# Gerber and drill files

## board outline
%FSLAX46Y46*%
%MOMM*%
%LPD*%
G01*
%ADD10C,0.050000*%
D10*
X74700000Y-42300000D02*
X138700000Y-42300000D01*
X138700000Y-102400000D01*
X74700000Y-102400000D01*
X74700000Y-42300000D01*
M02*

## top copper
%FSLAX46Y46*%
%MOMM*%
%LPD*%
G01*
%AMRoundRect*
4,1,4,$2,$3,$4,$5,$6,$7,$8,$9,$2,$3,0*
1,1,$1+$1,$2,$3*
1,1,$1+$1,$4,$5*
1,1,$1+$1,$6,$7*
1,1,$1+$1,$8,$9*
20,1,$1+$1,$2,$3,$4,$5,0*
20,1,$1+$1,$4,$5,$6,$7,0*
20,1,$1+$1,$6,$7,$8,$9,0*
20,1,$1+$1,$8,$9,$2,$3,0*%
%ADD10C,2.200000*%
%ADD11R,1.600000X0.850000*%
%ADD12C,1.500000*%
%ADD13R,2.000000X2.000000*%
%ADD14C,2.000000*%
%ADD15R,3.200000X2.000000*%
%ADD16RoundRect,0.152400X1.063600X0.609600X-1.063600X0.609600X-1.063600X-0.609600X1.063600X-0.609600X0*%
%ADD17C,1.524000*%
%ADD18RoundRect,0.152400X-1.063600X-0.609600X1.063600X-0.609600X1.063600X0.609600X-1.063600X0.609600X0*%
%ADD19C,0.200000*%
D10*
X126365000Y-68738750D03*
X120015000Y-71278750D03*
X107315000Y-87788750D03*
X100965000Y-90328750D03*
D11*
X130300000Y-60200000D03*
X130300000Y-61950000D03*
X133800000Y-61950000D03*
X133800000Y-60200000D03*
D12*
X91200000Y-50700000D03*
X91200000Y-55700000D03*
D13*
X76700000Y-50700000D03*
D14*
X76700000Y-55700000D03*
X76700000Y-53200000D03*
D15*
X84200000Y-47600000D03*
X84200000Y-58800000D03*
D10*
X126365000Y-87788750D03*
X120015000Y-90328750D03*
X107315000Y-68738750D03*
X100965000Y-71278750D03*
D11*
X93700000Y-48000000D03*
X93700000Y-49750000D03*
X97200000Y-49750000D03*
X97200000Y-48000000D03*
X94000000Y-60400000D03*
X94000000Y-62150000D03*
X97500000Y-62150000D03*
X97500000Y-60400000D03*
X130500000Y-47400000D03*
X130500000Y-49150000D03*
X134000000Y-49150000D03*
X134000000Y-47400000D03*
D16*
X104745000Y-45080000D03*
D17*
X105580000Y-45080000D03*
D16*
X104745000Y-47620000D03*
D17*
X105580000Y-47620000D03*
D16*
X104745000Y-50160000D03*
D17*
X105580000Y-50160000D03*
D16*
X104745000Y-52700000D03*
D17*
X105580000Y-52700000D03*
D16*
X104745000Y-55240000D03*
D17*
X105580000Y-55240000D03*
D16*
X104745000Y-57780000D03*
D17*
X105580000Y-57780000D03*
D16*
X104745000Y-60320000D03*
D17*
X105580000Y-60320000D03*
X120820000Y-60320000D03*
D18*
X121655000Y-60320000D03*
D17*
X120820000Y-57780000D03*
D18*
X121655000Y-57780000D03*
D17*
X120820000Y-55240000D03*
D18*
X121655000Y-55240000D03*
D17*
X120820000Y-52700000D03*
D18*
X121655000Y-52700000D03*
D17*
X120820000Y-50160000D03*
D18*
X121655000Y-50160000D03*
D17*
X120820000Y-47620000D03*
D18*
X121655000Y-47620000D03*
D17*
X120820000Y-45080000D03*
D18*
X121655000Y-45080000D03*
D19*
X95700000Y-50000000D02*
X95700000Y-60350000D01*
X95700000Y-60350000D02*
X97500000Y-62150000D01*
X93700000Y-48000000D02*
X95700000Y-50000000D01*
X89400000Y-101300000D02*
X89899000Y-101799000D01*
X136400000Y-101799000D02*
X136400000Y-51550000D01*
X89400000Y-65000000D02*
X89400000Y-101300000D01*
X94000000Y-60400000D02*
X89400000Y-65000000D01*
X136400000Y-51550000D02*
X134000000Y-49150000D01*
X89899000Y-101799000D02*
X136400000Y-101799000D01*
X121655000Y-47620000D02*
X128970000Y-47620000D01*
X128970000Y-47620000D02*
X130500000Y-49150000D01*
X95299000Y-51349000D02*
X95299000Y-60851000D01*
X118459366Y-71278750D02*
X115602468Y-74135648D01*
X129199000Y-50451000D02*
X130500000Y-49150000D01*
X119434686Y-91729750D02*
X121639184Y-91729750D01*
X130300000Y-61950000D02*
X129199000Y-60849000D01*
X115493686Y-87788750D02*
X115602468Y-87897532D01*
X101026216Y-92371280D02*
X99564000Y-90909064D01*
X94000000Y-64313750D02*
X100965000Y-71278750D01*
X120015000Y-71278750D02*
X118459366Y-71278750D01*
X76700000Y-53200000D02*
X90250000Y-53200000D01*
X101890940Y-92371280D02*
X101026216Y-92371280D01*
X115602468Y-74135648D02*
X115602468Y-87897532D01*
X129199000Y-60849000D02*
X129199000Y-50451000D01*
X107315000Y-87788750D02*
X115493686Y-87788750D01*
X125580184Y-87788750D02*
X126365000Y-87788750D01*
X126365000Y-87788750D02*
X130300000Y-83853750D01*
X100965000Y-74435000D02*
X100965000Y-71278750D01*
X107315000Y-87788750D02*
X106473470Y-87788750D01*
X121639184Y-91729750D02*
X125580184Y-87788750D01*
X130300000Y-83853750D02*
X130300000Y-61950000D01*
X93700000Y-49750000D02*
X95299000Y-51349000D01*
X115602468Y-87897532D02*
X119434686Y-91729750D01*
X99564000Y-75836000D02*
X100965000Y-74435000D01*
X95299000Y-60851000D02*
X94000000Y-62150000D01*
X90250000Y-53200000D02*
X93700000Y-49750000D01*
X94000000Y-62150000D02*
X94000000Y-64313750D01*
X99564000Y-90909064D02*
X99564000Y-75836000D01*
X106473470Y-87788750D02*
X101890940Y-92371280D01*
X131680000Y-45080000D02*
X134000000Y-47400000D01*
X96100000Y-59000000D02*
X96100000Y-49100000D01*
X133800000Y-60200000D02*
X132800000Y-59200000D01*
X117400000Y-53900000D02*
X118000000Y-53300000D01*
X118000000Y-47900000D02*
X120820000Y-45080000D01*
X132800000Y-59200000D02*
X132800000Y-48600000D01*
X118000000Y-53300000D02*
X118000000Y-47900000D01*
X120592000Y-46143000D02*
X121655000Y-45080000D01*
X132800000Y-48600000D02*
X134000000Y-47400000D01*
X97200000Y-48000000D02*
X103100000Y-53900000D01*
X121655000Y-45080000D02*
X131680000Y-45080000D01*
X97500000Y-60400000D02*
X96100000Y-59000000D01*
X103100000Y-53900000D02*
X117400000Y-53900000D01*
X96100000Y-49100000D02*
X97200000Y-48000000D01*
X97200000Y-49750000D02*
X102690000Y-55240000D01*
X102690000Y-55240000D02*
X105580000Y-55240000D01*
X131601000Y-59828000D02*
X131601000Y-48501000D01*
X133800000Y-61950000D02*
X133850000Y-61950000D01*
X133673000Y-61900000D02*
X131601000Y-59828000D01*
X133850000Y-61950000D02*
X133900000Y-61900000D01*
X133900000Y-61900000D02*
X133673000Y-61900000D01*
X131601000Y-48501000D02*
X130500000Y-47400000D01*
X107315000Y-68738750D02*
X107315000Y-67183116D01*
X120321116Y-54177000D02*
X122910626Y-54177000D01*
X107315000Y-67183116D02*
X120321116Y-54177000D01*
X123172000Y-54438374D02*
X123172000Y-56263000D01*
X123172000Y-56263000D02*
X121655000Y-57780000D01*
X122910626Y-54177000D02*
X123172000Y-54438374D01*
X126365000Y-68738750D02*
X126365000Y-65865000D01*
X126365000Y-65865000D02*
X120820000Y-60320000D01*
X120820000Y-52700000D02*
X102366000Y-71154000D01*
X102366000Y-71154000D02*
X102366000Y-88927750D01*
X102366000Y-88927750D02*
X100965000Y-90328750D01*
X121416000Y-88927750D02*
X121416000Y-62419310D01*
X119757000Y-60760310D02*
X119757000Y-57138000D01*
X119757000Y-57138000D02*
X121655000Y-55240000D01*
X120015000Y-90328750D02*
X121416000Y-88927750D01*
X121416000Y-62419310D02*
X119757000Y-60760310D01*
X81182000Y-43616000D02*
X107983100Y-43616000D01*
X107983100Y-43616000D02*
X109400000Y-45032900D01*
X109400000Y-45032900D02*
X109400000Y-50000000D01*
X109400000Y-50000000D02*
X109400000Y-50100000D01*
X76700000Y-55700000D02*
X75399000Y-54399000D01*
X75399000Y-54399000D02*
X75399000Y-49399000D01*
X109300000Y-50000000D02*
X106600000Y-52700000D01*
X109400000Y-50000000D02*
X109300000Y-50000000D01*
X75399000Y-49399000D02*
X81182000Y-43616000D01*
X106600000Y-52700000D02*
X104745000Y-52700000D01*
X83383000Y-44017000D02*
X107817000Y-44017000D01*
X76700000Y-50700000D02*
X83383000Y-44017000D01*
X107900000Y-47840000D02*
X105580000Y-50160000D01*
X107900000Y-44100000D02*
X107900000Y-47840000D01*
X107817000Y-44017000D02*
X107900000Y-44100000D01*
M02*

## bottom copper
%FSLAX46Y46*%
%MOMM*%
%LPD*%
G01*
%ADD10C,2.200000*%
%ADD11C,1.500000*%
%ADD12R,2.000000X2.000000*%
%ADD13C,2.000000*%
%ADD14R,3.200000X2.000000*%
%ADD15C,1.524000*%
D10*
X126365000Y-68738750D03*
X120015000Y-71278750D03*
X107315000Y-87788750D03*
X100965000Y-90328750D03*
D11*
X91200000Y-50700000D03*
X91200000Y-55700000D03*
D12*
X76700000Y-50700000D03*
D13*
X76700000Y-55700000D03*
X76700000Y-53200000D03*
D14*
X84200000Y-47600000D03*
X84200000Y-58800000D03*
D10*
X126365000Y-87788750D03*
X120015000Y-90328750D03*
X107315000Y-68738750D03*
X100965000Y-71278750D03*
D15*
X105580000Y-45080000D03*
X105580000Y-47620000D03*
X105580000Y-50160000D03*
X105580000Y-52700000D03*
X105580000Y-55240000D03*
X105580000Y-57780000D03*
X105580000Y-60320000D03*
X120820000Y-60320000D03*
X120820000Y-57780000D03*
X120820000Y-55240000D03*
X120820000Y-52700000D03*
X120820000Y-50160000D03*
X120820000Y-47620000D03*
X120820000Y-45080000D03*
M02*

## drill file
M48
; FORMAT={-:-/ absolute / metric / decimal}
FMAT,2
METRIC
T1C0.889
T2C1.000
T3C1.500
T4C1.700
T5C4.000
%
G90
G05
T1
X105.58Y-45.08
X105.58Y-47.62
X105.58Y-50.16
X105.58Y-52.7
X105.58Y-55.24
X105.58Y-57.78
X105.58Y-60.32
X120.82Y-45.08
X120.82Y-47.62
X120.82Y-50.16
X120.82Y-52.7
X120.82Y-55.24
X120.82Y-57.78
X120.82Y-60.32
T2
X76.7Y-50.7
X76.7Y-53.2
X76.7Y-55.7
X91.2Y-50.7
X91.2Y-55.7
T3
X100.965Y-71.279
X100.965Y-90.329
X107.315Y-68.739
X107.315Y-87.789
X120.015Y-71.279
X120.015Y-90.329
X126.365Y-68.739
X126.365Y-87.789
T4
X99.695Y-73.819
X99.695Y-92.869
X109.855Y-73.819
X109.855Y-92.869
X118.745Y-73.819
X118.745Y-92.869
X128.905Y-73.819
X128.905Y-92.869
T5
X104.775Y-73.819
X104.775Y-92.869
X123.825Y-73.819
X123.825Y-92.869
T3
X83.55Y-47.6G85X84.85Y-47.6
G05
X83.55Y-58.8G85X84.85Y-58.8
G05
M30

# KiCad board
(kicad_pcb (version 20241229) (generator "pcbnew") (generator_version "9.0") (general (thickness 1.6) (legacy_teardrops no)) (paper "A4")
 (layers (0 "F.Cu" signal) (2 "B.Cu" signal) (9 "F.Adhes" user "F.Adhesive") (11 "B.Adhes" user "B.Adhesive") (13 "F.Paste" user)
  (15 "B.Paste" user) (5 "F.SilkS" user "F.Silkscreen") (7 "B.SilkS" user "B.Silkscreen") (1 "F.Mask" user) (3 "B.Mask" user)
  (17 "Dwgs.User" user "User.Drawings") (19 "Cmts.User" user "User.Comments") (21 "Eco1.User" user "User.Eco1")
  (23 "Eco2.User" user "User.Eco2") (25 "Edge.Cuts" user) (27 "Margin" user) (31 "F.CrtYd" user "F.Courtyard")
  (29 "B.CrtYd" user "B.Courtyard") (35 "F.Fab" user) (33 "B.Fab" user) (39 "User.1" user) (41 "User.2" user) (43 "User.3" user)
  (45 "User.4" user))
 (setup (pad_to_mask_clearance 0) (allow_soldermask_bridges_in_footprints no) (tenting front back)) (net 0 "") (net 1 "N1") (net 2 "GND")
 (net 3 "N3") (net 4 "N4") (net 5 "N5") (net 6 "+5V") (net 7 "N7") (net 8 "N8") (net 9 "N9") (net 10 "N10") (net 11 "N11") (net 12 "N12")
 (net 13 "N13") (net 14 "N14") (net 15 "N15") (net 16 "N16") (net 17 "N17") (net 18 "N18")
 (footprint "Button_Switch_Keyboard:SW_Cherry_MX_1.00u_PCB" (layer "F.Cu") (at 126.365 68.73875)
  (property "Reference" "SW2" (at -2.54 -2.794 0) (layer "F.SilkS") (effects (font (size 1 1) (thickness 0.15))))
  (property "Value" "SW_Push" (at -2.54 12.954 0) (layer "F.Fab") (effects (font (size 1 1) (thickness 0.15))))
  (pad "" np_thru_hole circle (at -7.62 5.08) (size 1.7 1.7) (drill 1.7) (layers "*.Cu" "*.Mask"))
  (pad "" np_thru_hole circle (at -2.54 5.08) (size 4 4) (drill 4) (layers "*.Cu" "*.Mask"))
  (pad "" np_thru_hole circle (at 2.54 5.08) (size 1.7 1.7) (drill 1.7) (layers "*.Cu" "*.Mask"))
  (pad "1" thru_hole circle (at 0 0) (size 2.2 2.2) (drill 1.5) (layers "*.Cu" "*.Mask") (remove_unused_layers no) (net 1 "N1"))
  (pad "2" thru_hole circle (at -6.35 2.54) (size 2.2 2.2) (drill 1.5) (layers "*.Cu" "*.Mask") (remove_unused_layers no) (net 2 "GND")))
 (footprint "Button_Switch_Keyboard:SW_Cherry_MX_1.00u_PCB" (layer "F.Cu") (at 107.315 87.78875)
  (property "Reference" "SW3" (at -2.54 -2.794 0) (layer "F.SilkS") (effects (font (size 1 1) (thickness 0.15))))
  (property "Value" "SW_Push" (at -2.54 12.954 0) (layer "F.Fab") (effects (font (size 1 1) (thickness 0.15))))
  (pad "" np_thru_hole circle (at -7.62 5.08) (size 1.7 1.7) (drill 1.7) (layers "*.Cu" "*.Mask"))
  (pad "" np_thru_hole circle (at -2.54 5.08) (size 4 4) (drill 4) (layers "*.Cu" "*.Mask"))
  (pad "" np_thru_hole circle (at 2.54 5.08) (size 1.7 1.7) (drill 1.7) (layers "*.Cu" "*.Mask"))
  (pad "1" thru_hole circle (at 0 0) (size 2.2 2.2) (drill 1.5) (layers "*.Cu" "*.Mask") (remove_unused_layers no) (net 2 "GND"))
  (pad "2" thru_hole circle (at -6.35 2.54) (size 2.2 2.2) (drill 1.5) (layers "*.Cu" "*.Mask") (remove_unused_layers no) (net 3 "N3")))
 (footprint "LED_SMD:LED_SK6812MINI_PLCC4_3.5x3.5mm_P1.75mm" (layer "F.Cu") (at 132.05 61.075)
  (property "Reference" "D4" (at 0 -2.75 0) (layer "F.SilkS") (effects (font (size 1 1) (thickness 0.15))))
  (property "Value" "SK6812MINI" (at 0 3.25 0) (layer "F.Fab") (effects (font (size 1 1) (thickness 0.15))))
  (pad "1" smd rect (at -1.75 -0.875) (size 1.6 0.85) (layers "F.Cu" "F.Mask" "F.Paste") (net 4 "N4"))
  (pad "2" smd rect (at -1.75 0.875) (size 1.6 0.85) (layers "F.Cu" "F.Mask" "F.Paste") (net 2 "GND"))
  (pad "3" smd rect (at 1.75 0.875) (size 1.6 0.85) (layers "F.Cu" "F.Mask" "F.Paste") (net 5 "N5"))
  (pad "4" smd rect (at 1.75 -0.875) (size 1.6 0.85) (layers "F.Cu" "F.Mask" "F.Paste") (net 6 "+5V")))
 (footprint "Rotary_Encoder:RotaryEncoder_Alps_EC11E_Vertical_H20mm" (layer "F.Cu") (at 76.7 50.7)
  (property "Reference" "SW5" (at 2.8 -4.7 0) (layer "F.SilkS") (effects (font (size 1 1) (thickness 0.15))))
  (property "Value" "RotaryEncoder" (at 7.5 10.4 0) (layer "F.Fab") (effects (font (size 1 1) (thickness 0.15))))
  (pad "" thru_hole circle (at 14.5 0) (size 1.5 1.5) (drill 1) (layers "*.Cu" "*.Mask") (remove_unused_layers no))
  (pad "" thru_hole circle (at 14.5 5) (size 1.5 1.5) (drill 1) (layers "*.Cu" "*.Mask") (remove_unused_layers no))
  (pad "A" thru_hole rect (at 0 0) (size 2 2) (drill 1) (layers "*.Cu" "*.Mask") (remove_unused_layers no) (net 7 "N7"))
  (pad "B" thru_hole circle (at 0 5) (size 2 2) (drill 1) (layers "*.Cu" "*.Mask") (remove_unused_layers no) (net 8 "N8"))
  (pad "C" thru_hole circle (at 0 2.5) (size 2 2) (drill 1) (layers "*.Cu" "*.Mask") (remove_unused_layers no) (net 2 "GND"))
  (pad "MP" thru_hole rect (at 7.5 -3.1) (size 3.2 2) (drill oval 2.8 1.5) (layers "*.Cu" "*.Mask") (remove_unused_layers no))
  (pad "MP" thru_hole rect (at 7.5 8.1) (size 3.2 2) (drill oval 2.8 1.5) (layers "*.Cu" "*.Mask") (remove_unused_layers no)))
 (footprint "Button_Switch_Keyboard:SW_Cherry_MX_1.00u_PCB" (layer "F.Cu") (at 126.365 87.78875)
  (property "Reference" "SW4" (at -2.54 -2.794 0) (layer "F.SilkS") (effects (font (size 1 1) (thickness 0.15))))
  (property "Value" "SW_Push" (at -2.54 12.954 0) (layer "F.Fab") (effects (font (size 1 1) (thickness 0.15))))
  (pad "" np_thru_hole circle (at -7.62 5.08) (size 1.7 1.7) (drill 1.7) (layers "*.Cu" "*.Mask"))
  (pad "" np_thru_hole circle (at -2.54 5.08) (size 4 4) (drill 4) (layers "*.Cu" "*.Mask"))
  (pad "" np_thru_hole circle (at 2.54 5.08) (size 1.7 1.7) (drill 1.7) (layers "*.Cu" "*.Mask"))
  (pad "1" thru_hole circle (at 0 0) (size 2.2 2.2) (drill 1.5) (layers "*.Cu" "*.Mask") (remove_unused_layers no) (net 2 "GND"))
  (pad "2" thru_hole circle (at -6.35 2.54) (size 2.2 2.2) (drill 1.5) (layers "*.Cu" "*.Mask") (remove_unused_layers no) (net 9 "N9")))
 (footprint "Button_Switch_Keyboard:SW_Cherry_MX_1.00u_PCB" (layer "F.Cu") (at 107.315 68.73875)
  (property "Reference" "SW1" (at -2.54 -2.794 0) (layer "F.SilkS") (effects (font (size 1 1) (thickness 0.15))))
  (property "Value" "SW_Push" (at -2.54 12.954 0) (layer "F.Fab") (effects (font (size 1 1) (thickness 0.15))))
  (pad "" np_thru_hole circle (at -7.62 5.08) (size 1.7 1.7) (drill 1.7) (layers "*.Cu" "*.Mask"))
  (pad "" np_thru_hole circle (at -2.54 5.08) (size 4 4) (drill 4) (layers "*.Cu" "*.Mask"))
  (pad "" np_thru_hole circle (at 2.54 5.08) (size 1.7 1.7) (drill 1.7) (layers "*.Cu" "*.Mask"))
  (pad "1" thru_hole circle (at 0 0) (size 2.2 2.2) (drill 1.5) (layers "*.Cu" "*.Mask") (remove_unused_layers no) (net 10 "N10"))
  (pad "2" thru_hole circle (at -6.35 2.54) (size 2.2 2.2) (drill 1.5) (layers "*.Cu" "*.Mask") (remove_unused_layers no) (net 2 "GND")))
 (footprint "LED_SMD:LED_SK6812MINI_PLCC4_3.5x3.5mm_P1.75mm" (layer "F.Cu") (at 95.45 48.875)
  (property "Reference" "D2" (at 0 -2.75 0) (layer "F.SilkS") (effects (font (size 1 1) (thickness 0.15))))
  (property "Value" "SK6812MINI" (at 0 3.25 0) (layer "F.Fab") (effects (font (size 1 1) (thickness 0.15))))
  (pad "1" smd rect (at -1.75 -0.875) (size 1.6 0.85) (layers "F.Cu" "F.Mask" "F.Paste") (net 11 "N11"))
  (pad "2" smd rect (at -1.75 0.875) (size 1.6 0.85) (layers "F.Cu" "F.Mask" "F.Paste") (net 2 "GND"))
  (pad "3" smd rect (at 1.75 0.875) (size 1.6 0.85) (layers "F.Cu" "F.Mask" "F.Paste") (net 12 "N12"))
  (pad "4" smd rect (at 1.75 -0.875) (size 1.6 0.85) (layers "F.Cu" "F.Mask" "F.Paste") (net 6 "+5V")))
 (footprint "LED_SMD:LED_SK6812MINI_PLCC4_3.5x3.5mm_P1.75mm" (layer "F.Cu") (at 95.75 61.275)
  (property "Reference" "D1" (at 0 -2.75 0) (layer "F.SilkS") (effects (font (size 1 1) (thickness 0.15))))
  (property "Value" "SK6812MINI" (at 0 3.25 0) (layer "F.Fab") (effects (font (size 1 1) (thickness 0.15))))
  (pad "1" smd rect (at -1.75 -0.875) (size 1.6 0.85) (layers "F.Cu" "F.Mask" "F.Paste") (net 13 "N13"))
  (pad "2" smd rect (at -1.75 0.875) (size 1.6 0.85) (layers "F.Cu" "F.Mask" "F.Paste") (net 2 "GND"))
  (pad "3" smd rect (at 1.75 0.875) (size 1.6 0.85) (layers "F.Cu" "F.Mask" "F.Paste") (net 11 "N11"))
  (pad "4" smd rect (at 1.75 -0.875) (size 1.6 0.85) (layers "F.Cu" "F.Mask" "F.Paste") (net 6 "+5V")))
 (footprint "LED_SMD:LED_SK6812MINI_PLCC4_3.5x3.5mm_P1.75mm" (layer "F.Cu") (at 132.25 48.275)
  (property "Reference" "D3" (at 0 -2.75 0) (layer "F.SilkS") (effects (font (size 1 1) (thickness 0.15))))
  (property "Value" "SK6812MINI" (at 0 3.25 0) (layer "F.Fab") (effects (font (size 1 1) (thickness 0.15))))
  (pad "1" smd rect (at -1.75 -0.875) (size 1.6 0.85) (layers "F.Cu" "F.Mask" "F.Paste") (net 5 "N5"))
  (pad "2" smd rect (at -1.75 0.875) (size 1.6 0.85) (layers "F.Cu" "F.Mask" "F.Paste") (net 2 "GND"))
  (pad "3" smd rect (at 1.75 0.875) (size 1.6 0.85) (layers "F.Cu" "F.Mask" "F.Paste") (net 13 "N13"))
  (pad "4" smd rect (at 1.75 -0.875) (size 1.6 0.85) (layers "F.Cu" "F.Mask" "F.Paste") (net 6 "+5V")))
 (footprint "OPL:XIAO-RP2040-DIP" (layer "F.Cu") (at 113.2 52.7)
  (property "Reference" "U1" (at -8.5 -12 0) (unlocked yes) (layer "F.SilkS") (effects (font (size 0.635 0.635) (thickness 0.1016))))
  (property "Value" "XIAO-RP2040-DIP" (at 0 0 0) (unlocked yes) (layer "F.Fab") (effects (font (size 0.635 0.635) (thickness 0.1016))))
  (pad "1" smd roundrect (at -8.455 -7.62 180) (size 2.432 1.524) (layers "F.Cu" "F.Mask") (roundrect_rratio 0.1) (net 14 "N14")
   (thermal_bridge_angle 45))
  (pad "1" thru_hole circle (at -7.62 -7.62 180) (size 1.524 1.524) (drill 0.889) (layers "*.Cu" "*.Mask") (remove_unused_layers no)
   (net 14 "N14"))
  (pad "2" smd roundrect (at -8.455 -5.08 180) (size 2.432 1.524) (layers "F.Cu" "F.Mask") (roundrect_rratio 0.1) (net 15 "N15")
   (thermal_bridge_angle 45))
  (pad "2" thru_hole circle (at -7.62 -5.08 180) (size 1.524 1.524) (drill 0.889) (layers "*.Cu" "*.Mask") (remove_unused_layers no)
   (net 15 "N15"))
  (pad "3" smd roundrect (at -8.455 -2.54 180) (size 2.432 1.524) (layers "F.Cu" "F.Mask") (roundrect_rratio 0.1) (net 7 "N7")
   (thermal_bridge_angle 45))
  (pad "3" thru_hole circle (at -7.62 -2.54 180) (size 1.524 1.524) (drill 0.889) (layers "*.Cu" "*.Mask") (remove_unused_layers no)
   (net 7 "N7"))
  (pad "4" smd roundrect (at -8.455 0 180) (size 2.432 1.524) (layers "F.Cu" "F.Mask") (roundrect_rratio 0.1) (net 8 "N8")
   (thermal_bridge_angle 45))
  (pad "4" thru_hole circle (at -7.62 0 180) (size 1.524 1.524) (drill 0.889) (layers "*.Cu" "*.Mask") (remove_unused_layers no)
   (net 8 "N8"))
  (pad "5" smd roundrect (at -8.455 2.54 180) (size 2.432 1.524) (layers "F.Cu" "F.Mask") (roundrect_rratio 0.1) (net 12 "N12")
   (thermal_bridge_angle 45))
  (pad "5" thru_hole circle (at -7.62 2.54 180) (size 1.524 1.524) (drill 0.889) (layers "*.Cu" "*.Mask") (remove_unused_layers no)
   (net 12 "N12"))
  (pad "6" smd roundrect (at -8.455 5.08 180) (size 2.432 1.524) (layers "F.Cu" "F.Mask") (roundrect_rratio 0.1) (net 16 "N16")
   (thermal_bridge_angle 45))
  (pad "6" thru_hole circle (at -7.62 5.08 180) (size 1.524 1.524) (drill 0.889) (layers "*.Cu" "*.Mask") (remove_unused_layers no)
   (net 16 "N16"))
  (pad "7" smd roundrect (at -8.455 7.62 180) (size 2.432 1.524) (layers "F.Cu" "F.Mask") (roundrect_rratio 0.1) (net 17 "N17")
   (thermal_bridge_angle 45))
  (pad "7" thru_hole circle (at -7.62 7.62 180) (size 1.524 1.524) (drill 0.889) (layers "*.Cu" "*.Mask") (remove_unused_layers no)
   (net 17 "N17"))
  (pad "8" thru_hole circle (at 7.62 7.62) (size 1.524 1.524) (drill 0.889) (layers "*.Cu" "*.Mask") (remove_unused_layers no) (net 1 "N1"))
  (pad "8" smd roundrect (at 8.455 7.62) (size 2.432 1.524) (layers "F.Cu" "F.Mask") (roundrect_rratio 0.1) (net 1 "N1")
   (thermal_bridge_angle 45))
  (pad "9" thru_hole circle (at 7.62 5.08) (size 1.524 1.524) (drill 0.889) (layers "*.Cu" "*.Mask") (remove_unused_layers no)
   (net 10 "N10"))
  (pad "9" smd roundrect (at 8.455 5.08) (size 2.432 1.524) (layers "F.Cu" "F.Mask") (roundrect_rratio 0.1) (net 10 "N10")
   (thermal_bridge_angle 45))
  (pad "10" thru_hole circle (at 7.62 2.54) (size 1.524 1.524) (drill 0.889) (layers "*.Cu" "*.Mask") (remove_unused_layers no) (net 9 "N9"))
  (pad "10" smd roundrect (at 8.455 2.54) (size 2.432 1.524) (layers "F.Cu" "F.Mask") (roundrect_rratio 0.1) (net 9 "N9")
   (thermal_bridge_angle 45))
  (pad "11" thru_hole circle (at 7.62 0) (size 1.524 1.524) (drill 0.889) (layers "*.Cu" "*.Mask") (remove_unused_layers no) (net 3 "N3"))
  (pad "11" smd roundrect (at 8.455 0) (size 2.432 1.524) (layers "F.Cu" "F.Mask") (roundrect_rratio 0.1) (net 3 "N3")
   (thermal_bridge_angle 45))
  (pad "12" thru_hole circle (at 7.62 -2.54) (size 1.524 1.524) (drill 0.889) (layers "*.Cu" "*.Mask") (remove_unused_layers no)
   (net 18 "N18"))
  (pad "12" smd roundrect (at 8.455 -2.54) (size 2.432 1.524) (layers "F.Cu" "F.Mask") (roundrect_rratio 0.1) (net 18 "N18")
   (thermal_bridge_angle 45))
  (pad "13" thru_hole circle (at 7.62 -5.08) (size 1.524 1.524) (drill 0.889) (layers "*.Cu" "*.Mask") (remove_unused_layers no)
   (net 2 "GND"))
  (pad "13" smd roundrect (at 8.455 -5.08) (size 2.432 1.524) (layers "F.Cu" "F.Mask") (roundrect_rratio 0.1) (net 2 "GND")
   (thermal_bridge_angle 45))
  (pad "14" thru_hole circle (at 7.62 -7.62) (size 1.524 1.524) (drill 0.889) (layers "*.Cu" "*.Mask") (remove_unused_layers no)
   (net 6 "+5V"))
  (pad "14" smd roundrect (at 8.455 -7.62) (size 2.432 1.524) (layers "F.Cu" "F.Mask") (roundrect_rratio 0.1) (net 6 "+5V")
   (thermal_bridge_angle 45)))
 (gr_rect (start 74.7 42.3) (end 138.7 102.4) (stroke (width 0.05) (type default)) (fill no) (layer "Edge.Cuts"))
 (segment (start 95.7 50) (end 95.7 60.35) (width 0.2) (layer "F.Cu") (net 11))
 (segment (start 95.7 60.35) (end 97.5 62.15) (width 0.2) (layer "F.Cu") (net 11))
 (segment (start 93.7 48) (end 95.7 50) (width 0.2) (layer "F.Cu") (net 11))
 (segment (start 89.4 101.3) (end 89.899 101.799) (width 0.2) (layer "F.Cu") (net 13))
 (segment (start 136.4 101.799) (end 136.4 51.55) (width 0.2) (layer "F.Cu") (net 13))
 (segment (start 89.4 65) (end 89.4 101.3) (width 0.2) (layer "F.Cu") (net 13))
 (segment (start 94 60.4) (end 89.4 65) (width 0.2) (layer "F.Cu") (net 13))
 (segment (start 136.4 51.55) (end 134 49.15) (width 0.2) (layer "F.Cu") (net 13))
 (segment (start 89.899 101.799) (end 136.4 101.799) (width 0.2) (layer "F.Cu") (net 13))
 (segment (start 121.655 47.62) (end 128.97 47.62) (width 0.2) (layer "F.Cu") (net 2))
 (segment (start 128.97 47.62) (end 130.5 49.15) (width 0.2) (layer "F.Cu") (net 2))
 (segment (start 95.299 51.349) (end 95.299 60.851) (width 0.2) (layer "F.Cu") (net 2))
 (segment (start 118.459366 71.27875) (end 115.602468 74.135648) (width 0.2) (layer "F.Cu") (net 2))
 (segment (start 129.199 50.451) (end 130.5 49.15) (width 0.2) (layer "F.Cu") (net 2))
 (segment (start 119.434686 91.72975) (end 121.639184 91.72975) (width 0.2) (layer "F.Cu") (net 2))
 (segment (start 130.3 61.95) (end 129.199 60.849) (width 0.2) (layer "F.Cu") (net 2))
 (segment (start 115.493686 87.78875) (end 115.602468 87.897532) (width 0.2) (layer "F.Cu") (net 2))
 (segment (start 101.026216 92.37128) (end 99.564 90.909064) (width 0.2) (layer "F.Cu") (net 2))
 (segment (start 94 64.31375) (end 100.965 71.27875) (width 0.2) (layer "F.Cu") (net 2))
 (segment (start 120.015 71.27875) (end 118.459366 71.27875) (width 0.2) (layer "F.Cu") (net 2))
 (segment (start 76.7 53.2) (end 90.25 53.2) (width 0.2) (layer "F.Cu") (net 2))
 (segment (start 101.89094 92.37128) (end 101.026216 92.37128) (width 0.2) (layer "F.Cu") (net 2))
 (segment (start 115.602468 74.135648) (end 115.602468 87.897532) (width 0.2) (layer "F.Cu") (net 2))
 (segment (start 129.199 60.849) (end 129.199 50.451) (width 0.2) (layer "F.Cu") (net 2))
 (segment (start 107.315 87.78875) (end 115.493686 87.78875) (width 0.2) (layer "F.Cu") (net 2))
 (segment (start 125.580184 87.78875) (end 126.365 87.78875) (width 0.2) (layer "F.Cu") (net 2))
 (segment (start 126.365 87.78875) (end 130.3 83.85375) (width 0.2) (layer "F.Cu") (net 2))
 (segment (start 100.965 74.435) (end 100.965 71.27875) (width 0.2) (layer "F.Cu") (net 2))
 (segment (start 107.315 87.78875) (end 106.47347 87.78875) (width 0.2) (layer "F.Cu") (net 2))
 (segment (start 121.639184 91.72975) (end 125.580184 87.78875) (width 0.2) (layer "F.Cu") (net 2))
 (segment (start 130.3 83.85375) (end 130.3 61.95) (width 0.2) (layer "F.Cu") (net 2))
 (segment (start 93.7 49.75) (end 95.299 51.349) (width 0.2) (layer "F.Cu") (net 2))
 (segment (start 115.602468 87.897532) (end 119.434686 91.72975) (width 0.2) (layer "F.Cu") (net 2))
 (segment (start 99.564 75.836) (end 100.965 74.435) (width 0.2) (layer "F.Cu") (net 2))
 (segment (start 95.299 60.851) (end 94 62.15) (width 0.2) (layer "F.Cu") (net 2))
 (segment (start 90.25 53.2) (end 93.7 49.75) (width 0.2) (layer "F.Cu") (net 2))
 (segment (start 94 62.15) (end 94 64.31375) (width 0.2) (layer "F.Cu") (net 2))
 (segment (start 99.564 90.909064) (end 99.564 75.836) (width 0.2) (layer "F.Cu") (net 2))
 (segment (start 106.47347 87.78875) (end 101.89094 92.37128) (width 0.2) (layer "F.Cu") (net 2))
 (segment (start 131.68 45.08) (end 134 47.4) (width 0.2) (layer "F.Cu") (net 6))
 (segment (start 96.1 59) (end 96.1 49.1) (width 0.2) (layer "F.Cu") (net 6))
 (segment (start 133.8 60.2) (end 132.8 59.2) (width 0.2) (layer "F.Cu") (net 6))
 (segment (start 117.4 53.9) (end 118 53.3) (width 0.2) (layer "F.Cu") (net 6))
 (segment (start 118 47.9) (end 120.82 45.08) (width 0.2) (layer "F.Cu") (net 6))
 (segment (start 132.8 59.2) (end 132.8 48.6) (width 0.2) (layer "F.Cu") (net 6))
 (segment (start 118 53.3) (end 118 47.9) (width 0.2) (layer "F.Cu") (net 6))
 (segment (start 120.592 46.143) (end 121.655 45.08) (width 0.2) (layer "F.Cu") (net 6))
 (segment (start 132.8 48.6) (end 134 47.4) (width 0.2) (layer "F.Cu") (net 6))
 (segment (start 97.2 48) (end 103.1 53.9) (width 0.2) (layer "F.Cu") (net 6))
 (segment (start 121.655 45.08) (end 131.68 45.08) (width 0.2) (layer "F.Cu") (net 6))
 (segment (start 97.5 60.4) (end 96.1 59) (width 0.2) (layer "F.Cu") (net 6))
 (segment (start 103.1 53.9) (end 117.4 53.9) (width 0.2) (layer "F.Cu") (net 6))
 (segment (start 96.1 49.1) (end 97.2 48) (width 0.2) (layer "F.Cu") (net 6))
 (segment (start 97.2 49.75) (end 102.69 55.24) (width 0.2) (layer "F.Cu") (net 12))
 (segment (start 102.69 55.24) (end 105.58 55.24) (width 0.2) (layer "F.Cu") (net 12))
 (segment (start 131.601 59.828) (end 131.601 48.501) (width 0.2) (layer "F.Cu") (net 5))
 (segment (start 133.8 61.95) (end 133.85 61.95) (width 0.2) (layer "F.Cu") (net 5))
 (segment (start 133.673 61.9) (end 131.601 59.828) (width 0.2) (layer "F.Cu") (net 5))
 (segment (start 133.85 61.95) (end 133.9 61.9) (width 0.2) (layer "F.Cu") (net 5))
 (segment (start 133.9 61.9) (end 133.673 61.9) (width 0.2) (layer "F.Cu") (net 5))
 (segment (start 131.601 48.501) (end 130.5 47.4) (width 0.2) (layer "F.Cu") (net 5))
 (segment (start 107.315 68.73875) (end 107.315 67.183116) (width 0.2) (layer "F.Cu") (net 10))
 (segment (start 120.321116 54.177) (end 122.910626 54.177) (width 0.2) (layer "F.Cu") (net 10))
 (segment (start 107.315 67.183116) (end 120.321116 54.177) (width 0.2) (layer "F.Cu") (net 10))
 (segment (start 123.172 54.438374) (end 123.172 56.263) (width 0.2) (layer "F.Cu") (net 10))
 (segment (start 123.172 56.263) (end 121.655 57.78) (width 0.2) (layer "F.Cu") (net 10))
 (segment (start 122.910626 54.177) (end 123.172 54.438374) (width 0.2) (layer "F.Cu") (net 10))
 (segment (start 126.365 68.73875) (end 126.365 65.865) (width 0.2) (layer "F.Cu") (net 1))
 (segment (start 126.365 65.865) (end 120.82 60.32) (width 0.2) (layer "F.Cu") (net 1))
 (segment (start 120.82 52.7) (end 102.366 71.154) (width 0.2) (layer "F.Cu") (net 3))
 (segment (start 102.366 71.154) (end 102.366 88.92775) (width 0.2) (layer "F.Cu") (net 3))
 (segment (start 102.366 88.92775) (end 100.965 90.32875) (width 0.2) (layer "F.Cu") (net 3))
 (segment (start 121.416 88.92775) (end 121.416 62.41931) (width 0.2) (layer "F.Cu") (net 9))
 (segment (start 119.757 60.76031) (end 119.757 57.138) (width 0.2) (layer "F.Cu") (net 9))
 (segment (start 119.757 57.138) (end 121.655 55.24) (width 0.2) (layer "F.Cu") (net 9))
 (segment (start 120.015 90.32875) (end 121.416 88.92775) (width 0.2) (layer "F.Cu") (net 9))
 (segment (start 121.416 62.41931) (end 119.757 60.76031) (width 0.2) (layer "F.Cu") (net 9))
 (segment (start 81.182 43.616) (end 107.9831 43.616) (width 0.2) (layer "F.Cu") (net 8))
 (segment (start 107.9831 43.616) (end 109.4 45.0329) (width 0.2) (layer "F.Cu") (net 8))
 (segment (start 109.4 45.0329) (end 109.4 50) (width 0.2) (layer "F.Cu") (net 8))
 (segment (start 109.4 50) (end 109.4 50.1) (width 0.2) (layer "F.Cu") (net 8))
 (segment (start 76.7 55.7) (end 75.399 54.399) (width 0.2) (layer "F.Cu") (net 8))
 (segment (start 75.399 54.399) (end 75.399 49.399) (width 0.2) (layer "F.Cu") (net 8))
 (segment (start 109.3 50) (end 106.6 52.7) (width 0.2) (layer "F.Cu") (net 8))
 (segment (start 109.4 50) (end 109.3 50) (width 0.2) (layer "F.Cu") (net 8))
 (segment (start 75.399 49.399) (end 81.182 43.616) (width 0.2) (layer "F.Cu") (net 8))
 (segment (start 106.6 52.7) (end 104.745 52.7) (width 0.2) (layer "F.Cu") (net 8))
 (segment (start 83.383 44.017) (end 107.817 44.017) (width 0.2) (layer "F.Cu") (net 7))
 (segment (start 76.7 50.7) (end 83.383 44.017) (width 0.2) (layer "F.Cu") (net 7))
 (segment (start 107.9 47.84) (end 105.58 50.16) (width 0.2) (layer "F.Cu") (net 7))
 (segment (start 107.9 44.1) (end 107.9 47.84) (width 0.2) (layer "F.Cu") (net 7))
 (segment (start 107.817 44.017) (end 107.9 44.1) (width 0.2) (layer "F.Cu") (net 7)))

